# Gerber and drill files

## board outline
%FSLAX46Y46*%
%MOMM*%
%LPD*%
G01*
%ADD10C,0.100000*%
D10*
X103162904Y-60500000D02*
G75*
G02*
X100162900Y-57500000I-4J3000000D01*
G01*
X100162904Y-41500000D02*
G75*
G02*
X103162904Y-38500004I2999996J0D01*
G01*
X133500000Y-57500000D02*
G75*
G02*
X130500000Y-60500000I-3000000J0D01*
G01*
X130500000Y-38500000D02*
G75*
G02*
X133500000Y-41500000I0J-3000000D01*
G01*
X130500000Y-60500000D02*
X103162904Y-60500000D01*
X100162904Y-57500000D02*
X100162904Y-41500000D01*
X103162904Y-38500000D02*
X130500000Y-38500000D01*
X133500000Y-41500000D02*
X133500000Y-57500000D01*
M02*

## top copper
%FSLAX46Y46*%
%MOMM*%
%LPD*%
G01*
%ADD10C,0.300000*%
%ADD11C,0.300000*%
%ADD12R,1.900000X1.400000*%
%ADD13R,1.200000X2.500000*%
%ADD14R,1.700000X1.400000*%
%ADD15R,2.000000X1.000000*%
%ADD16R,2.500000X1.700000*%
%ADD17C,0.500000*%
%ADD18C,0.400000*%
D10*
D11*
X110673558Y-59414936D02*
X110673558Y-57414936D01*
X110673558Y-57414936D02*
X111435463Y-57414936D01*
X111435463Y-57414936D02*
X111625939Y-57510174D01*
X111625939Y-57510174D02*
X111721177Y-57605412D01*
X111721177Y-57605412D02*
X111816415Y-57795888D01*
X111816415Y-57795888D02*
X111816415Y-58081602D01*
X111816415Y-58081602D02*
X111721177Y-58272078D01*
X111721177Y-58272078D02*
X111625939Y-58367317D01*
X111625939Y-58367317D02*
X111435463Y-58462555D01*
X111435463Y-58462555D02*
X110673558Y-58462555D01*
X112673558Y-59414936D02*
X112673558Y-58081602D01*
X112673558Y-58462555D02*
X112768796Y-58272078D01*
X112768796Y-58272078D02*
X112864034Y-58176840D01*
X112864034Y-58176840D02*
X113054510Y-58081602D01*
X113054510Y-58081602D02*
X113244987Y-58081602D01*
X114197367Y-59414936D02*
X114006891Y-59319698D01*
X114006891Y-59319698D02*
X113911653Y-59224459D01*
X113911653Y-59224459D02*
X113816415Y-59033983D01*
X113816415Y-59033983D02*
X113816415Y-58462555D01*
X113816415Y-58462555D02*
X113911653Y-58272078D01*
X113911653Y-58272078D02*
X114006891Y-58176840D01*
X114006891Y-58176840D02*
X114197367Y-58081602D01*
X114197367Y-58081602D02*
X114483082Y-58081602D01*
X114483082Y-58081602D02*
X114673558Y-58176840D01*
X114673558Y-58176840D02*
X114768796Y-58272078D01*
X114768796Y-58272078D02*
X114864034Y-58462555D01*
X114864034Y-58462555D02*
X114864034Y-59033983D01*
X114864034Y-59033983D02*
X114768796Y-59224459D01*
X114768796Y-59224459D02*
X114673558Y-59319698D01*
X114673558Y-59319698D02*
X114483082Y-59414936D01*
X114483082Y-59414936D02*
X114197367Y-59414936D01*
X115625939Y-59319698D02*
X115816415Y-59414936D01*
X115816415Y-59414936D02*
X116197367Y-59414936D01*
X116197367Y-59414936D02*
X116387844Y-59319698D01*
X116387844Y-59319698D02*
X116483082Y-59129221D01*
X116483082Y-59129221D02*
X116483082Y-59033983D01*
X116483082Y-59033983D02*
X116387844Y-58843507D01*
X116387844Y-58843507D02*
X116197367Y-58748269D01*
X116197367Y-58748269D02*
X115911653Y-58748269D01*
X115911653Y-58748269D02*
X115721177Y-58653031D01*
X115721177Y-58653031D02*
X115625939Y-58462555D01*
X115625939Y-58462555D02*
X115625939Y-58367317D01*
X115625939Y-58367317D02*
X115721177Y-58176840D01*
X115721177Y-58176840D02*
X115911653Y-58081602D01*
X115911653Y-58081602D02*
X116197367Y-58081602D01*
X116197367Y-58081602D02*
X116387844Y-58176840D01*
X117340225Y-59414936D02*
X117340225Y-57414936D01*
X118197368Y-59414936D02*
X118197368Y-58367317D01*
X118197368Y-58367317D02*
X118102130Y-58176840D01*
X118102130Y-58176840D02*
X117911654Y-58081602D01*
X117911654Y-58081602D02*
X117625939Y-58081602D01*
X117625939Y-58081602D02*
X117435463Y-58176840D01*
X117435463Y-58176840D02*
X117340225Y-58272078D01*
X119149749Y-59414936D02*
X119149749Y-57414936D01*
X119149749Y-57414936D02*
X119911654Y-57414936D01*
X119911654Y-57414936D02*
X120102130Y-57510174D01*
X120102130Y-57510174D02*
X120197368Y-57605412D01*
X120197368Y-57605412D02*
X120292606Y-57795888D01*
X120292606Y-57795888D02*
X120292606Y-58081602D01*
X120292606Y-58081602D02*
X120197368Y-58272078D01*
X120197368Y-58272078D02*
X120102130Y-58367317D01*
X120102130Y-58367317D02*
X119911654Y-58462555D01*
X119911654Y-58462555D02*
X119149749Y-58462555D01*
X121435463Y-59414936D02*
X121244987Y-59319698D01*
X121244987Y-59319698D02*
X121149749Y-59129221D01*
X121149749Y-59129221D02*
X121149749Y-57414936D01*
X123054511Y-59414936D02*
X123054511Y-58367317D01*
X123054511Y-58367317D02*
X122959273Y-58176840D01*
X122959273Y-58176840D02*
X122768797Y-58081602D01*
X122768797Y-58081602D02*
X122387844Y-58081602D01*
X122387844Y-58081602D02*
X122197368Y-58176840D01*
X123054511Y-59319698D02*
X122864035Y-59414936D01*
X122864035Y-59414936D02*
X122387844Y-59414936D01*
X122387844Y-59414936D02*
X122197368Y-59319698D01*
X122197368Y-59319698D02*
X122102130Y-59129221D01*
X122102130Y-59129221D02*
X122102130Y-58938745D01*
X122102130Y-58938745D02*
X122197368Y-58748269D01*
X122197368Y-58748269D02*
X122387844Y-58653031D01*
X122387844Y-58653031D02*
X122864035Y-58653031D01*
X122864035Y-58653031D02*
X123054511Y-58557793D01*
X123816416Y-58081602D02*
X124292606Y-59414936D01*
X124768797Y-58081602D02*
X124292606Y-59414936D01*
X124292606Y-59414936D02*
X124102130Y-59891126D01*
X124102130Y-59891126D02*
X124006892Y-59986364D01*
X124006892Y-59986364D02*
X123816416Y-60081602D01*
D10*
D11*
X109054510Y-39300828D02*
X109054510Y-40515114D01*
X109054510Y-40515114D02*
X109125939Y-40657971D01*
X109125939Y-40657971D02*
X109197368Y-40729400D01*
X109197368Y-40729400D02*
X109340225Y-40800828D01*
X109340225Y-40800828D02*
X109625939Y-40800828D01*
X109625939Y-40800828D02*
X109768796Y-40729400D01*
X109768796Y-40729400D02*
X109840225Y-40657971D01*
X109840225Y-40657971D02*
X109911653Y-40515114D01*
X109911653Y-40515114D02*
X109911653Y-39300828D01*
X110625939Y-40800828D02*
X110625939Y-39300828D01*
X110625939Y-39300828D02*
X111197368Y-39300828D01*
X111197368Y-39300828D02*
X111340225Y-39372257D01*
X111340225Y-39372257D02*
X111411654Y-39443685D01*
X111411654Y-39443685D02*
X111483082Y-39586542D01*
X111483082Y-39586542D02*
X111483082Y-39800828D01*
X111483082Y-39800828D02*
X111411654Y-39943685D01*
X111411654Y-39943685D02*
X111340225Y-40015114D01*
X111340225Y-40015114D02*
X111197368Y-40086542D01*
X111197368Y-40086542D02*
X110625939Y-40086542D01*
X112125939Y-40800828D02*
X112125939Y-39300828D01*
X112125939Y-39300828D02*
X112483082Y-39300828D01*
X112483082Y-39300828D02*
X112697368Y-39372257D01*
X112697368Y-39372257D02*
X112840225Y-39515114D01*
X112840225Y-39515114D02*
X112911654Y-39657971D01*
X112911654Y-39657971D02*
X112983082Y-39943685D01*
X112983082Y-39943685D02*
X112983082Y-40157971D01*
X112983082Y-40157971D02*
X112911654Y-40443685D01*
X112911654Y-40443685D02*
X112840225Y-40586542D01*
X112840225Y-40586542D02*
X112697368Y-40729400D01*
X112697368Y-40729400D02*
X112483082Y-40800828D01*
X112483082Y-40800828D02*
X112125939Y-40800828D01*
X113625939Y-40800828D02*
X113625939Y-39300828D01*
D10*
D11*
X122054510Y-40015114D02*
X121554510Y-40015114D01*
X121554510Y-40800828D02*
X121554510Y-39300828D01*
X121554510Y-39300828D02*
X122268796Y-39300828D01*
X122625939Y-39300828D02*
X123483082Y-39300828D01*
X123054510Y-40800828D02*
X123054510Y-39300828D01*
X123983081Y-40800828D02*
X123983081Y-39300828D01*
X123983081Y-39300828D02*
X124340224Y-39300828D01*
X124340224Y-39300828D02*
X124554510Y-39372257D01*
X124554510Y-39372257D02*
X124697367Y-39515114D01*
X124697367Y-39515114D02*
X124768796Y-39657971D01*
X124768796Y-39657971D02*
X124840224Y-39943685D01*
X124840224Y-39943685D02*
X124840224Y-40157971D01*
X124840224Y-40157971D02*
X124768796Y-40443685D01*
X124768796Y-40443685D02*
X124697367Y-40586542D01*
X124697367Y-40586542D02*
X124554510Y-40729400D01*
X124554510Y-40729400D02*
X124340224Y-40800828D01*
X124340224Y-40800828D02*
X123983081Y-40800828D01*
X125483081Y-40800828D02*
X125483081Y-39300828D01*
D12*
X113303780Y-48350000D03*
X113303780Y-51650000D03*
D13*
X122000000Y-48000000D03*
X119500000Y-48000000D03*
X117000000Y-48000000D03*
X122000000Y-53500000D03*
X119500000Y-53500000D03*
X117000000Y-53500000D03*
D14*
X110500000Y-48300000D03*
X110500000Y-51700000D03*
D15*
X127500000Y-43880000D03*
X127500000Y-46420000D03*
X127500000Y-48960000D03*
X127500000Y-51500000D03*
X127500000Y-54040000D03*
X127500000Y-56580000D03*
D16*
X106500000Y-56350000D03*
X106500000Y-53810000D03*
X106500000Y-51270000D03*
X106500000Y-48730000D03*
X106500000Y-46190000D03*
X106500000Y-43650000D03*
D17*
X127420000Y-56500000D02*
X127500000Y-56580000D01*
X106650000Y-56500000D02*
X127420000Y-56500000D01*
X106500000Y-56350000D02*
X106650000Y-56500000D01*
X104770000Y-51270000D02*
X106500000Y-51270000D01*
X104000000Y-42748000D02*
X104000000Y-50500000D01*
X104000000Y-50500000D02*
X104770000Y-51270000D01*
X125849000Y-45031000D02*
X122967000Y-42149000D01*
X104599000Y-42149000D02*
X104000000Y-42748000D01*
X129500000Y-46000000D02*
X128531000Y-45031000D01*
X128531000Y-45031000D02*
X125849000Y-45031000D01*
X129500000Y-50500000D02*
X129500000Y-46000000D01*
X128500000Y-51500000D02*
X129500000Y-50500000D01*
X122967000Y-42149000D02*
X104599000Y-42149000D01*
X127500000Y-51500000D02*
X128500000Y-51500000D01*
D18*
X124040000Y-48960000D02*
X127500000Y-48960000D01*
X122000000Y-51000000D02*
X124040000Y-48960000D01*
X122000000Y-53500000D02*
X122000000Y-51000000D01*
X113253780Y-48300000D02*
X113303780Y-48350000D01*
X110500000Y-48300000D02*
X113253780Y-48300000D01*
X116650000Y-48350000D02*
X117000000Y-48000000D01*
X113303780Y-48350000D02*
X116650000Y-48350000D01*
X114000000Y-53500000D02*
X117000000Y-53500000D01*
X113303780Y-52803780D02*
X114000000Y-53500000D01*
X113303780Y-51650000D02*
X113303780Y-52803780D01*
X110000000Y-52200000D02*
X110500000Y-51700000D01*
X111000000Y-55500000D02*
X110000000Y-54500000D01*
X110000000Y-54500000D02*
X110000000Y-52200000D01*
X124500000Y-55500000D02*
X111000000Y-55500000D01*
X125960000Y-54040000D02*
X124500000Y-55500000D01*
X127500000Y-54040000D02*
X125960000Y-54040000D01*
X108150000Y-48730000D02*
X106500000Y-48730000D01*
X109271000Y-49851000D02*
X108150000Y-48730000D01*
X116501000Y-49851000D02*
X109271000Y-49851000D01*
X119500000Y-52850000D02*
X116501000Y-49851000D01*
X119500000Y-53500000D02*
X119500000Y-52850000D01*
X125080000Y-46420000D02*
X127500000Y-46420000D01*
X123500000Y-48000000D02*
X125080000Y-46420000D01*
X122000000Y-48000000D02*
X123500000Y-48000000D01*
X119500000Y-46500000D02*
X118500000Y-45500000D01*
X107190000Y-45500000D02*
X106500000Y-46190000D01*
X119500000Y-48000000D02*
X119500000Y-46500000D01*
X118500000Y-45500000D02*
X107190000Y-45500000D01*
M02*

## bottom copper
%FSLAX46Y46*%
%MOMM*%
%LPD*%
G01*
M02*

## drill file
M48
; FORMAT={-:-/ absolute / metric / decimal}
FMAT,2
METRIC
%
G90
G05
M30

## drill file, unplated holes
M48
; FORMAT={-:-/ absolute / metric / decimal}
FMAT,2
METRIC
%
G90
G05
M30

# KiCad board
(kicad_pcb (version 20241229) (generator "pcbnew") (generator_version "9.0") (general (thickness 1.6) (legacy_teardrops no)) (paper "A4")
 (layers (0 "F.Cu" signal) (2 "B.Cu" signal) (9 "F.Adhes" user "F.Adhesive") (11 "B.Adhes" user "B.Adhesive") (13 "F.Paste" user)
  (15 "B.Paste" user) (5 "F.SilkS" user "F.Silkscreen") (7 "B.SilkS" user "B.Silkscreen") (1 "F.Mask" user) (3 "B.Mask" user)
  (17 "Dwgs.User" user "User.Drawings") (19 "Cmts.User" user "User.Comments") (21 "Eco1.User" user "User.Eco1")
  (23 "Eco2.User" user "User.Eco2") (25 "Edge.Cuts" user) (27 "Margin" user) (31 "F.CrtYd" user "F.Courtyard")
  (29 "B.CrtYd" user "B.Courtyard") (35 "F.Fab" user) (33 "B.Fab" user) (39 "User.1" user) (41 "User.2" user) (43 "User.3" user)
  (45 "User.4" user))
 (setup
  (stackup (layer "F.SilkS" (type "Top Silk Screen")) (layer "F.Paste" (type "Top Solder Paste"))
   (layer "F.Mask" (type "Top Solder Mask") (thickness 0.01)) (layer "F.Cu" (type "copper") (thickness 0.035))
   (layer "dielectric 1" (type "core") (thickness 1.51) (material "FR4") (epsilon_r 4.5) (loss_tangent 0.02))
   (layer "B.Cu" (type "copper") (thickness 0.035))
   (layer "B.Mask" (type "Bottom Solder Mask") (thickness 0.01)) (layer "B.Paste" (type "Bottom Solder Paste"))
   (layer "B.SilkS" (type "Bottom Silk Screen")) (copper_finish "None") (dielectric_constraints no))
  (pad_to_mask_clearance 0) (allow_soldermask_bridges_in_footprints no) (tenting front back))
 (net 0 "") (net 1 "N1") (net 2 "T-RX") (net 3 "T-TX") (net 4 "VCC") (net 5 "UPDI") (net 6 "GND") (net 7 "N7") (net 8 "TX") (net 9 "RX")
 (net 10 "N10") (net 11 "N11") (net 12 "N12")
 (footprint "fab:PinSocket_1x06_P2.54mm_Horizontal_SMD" (layer "F.Cu") (at 127.5 43.88)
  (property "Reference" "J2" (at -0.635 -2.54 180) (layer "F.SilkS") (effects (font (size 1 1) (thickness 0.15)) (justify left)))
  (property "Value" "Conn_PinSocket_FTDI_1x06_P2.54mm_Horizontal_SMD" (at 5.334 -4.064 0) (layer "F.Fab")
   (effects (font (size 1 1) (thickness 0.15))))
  (pad "1" smd rect (at 0 0) (size 2 1) (layers "F.Cu" "F.Mask" "F.Paste") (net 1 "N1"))
  (pad "2" smd rect (at 0 2.54) (size 2 1) (layers "F.Cu" "F.Mask" "F.Paste") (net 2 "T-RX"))
  (pad "3" smd rect (at 0 5.08) (size 2 1) (layers "F.Cu" "F.Mask" "F.Paste") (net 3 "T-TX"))
  (pad "4" smd rect (at 0 7.62) (size 2 1) (layers "F.Cu" "F.Mask" "F.Paste") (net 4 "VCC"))
  (pad "5" smd rect (at 0 10.16) (size 2 1) (layers "F.Cu" "F.Mask" "F.Paste") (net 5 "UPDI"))
  (pad "6" smd rect (at 0 12.7) (size 2 1) (layers "F.Cu" "F.Mask" "F.Paste") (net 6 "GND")))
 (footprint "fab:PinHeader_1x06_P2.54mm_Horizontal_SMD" (layer "F.Cu") (at 106.5 56.35 180)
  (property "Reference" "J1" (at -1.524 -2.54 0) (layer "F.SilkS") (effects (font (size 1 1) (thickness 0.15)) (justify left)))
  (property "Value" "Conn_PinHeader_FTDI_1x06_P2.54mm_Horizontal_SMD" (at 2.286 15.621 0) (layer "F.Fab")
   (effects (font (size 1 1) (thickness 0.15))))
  (pad "1" smd rect (at 0 0 180) (size 2.5 1.7) (layers "F.Cu" "F.Mask" "F.Paste") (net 6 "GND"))
  (pad "2" smd rect (at 0 2.54 180) (size 2.5 1.7) (layers "F.Cu" "F.Mask" "F.Paste") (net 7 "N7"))
  (pad "3" smd rect (at 0 5.08 180) (size 2.5 1.7) (layers "F.Cu" "F.Mask" "F.Paste") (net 4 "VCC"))
  (pad "4" smd rect (at 0 7.62 180) (size 2.5 1.7) (layers "F.Cu" "F.Mask" "F.Paste") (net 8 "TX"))
  (pad "5" smd rect (at 0 10.16 180) (size 2.5 1.7) (layers "F.Cu" "F.Mask" "F.Paste") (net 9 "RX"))
  (pad "6" smd rect (at 0 12.7 180) (size 2.5 1.7) (layers "F.Cu" "F.Mask" "F.Paste") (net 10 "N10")))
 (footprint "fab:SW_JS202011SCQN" (layer "F.Cu") (at 119.5 50.75)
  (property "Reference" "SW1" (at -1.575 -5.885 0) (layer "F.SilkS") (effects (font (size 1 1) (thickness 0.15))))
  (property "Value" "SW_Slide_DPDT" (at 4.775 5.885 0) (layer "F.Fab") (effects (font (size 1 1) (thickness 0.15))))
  (pad "1" smd rect (at -2.5 2.75) (size 1.2 2.5) (layers "F.Cu" "F.Mask" "F.Paste") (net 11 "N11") (solder_mask_margin 0.102))
  (pad "2" smd rect (at 0 2.75) (size 1.2 2.5) (layers "F.Cu" "F.Mask" "F.Paste") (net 8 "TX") (solder_mask_margin 0.102))
  (pad "3" smd rect (at 2.5 2.75) (size 1.2 2.5) (layers "F.Cu" "F.Mask" "F.Paste") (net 3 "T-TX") (solder_mask_margin 0.102))
  (pad "4" smd rect (at 2.5 -2.75) (size 1.2 2.5) (layers "F.Cu" "F.Mask" "F.Paste") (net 2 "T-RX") (solder_mask_margin 0.102))
  (pad "5" smd rect (at 0 -2.75) (size 1.2 2.5) (layers "F.Cu" "F.Mask" "F.Paste") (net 9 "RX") (solder_mask_margin 0.102))
  (pad "6" smd rect (at -2.5 -2.75) (size 1.2 2.5) (layers "F.Cu" "F.Mask" "F.Paste") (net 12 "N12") (solder_mask_margin 0.102)))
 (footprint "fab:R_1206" (layer "F.Cu") (at 110.5 50 -90)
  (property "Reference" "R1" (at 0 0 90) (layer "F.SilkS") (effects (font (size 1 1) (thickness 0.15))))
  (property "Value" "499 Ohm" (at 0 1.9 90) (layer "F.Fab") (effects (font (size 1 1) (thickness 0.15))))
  (pad "1" smd rect (at -1.7 0 270) (size 1.4 1.7) (layers "F.Cu" "F.Mask" "F.Paste") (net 12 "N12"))
  (pad "2" smd rect (at 1.7 0 270) (size 1.4 1.7) (layers "F.Cu" "F.Mask" "F.Paste") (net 5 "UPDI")))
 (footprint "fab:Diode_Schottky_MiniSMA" (layer "F.Cu") (at 113.30378 50 90)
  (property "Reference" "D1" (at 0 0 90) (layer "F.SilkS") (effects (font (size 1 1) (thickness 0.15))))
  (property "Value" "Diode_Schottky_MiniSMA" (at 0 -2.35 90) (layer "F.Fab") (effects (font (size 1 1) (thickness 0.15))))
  (pad "1" smd rect (at -1.65 0 90) (size 1.4 1.9) (layers "F.Cu" "F.Mask" "F.Paste") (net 11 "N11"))
  (pad "2" smd rect (at 1.65 0 90) (size 1.4 1.9) (layers "F.Cu" "F.Mask" "F.Paste") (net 12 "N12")))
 (gr_line (start 103.162904 38.5) (end 130.5 38.5) (stroke (width 0.1) (type default)) (layer "Edge.Cuts"))
 (gr_line (start 130.5 60.5) (end 103.162904 60.5) (stroke (width 0.1) (type default)) (layer "Edge.Cuts"))
 (gr_line (start 100.162904 57.5) (end 100.162904 41.5) (stroke (width 0.1) (type default)) (layer "Edge.Cuts"))
 (gr_arc (start 133.5 57.5) (mid 132.62132 59.62132) (end 130.5 60.5) (stroke (width 0.1) (type default)) (layer "Edge.Cuts"))
 (gr_line (start 133.5 41.5) (end 133.5 57.5) (stroke (width 0.1) (type default)) (layer "Edge.Cuts"))
 (gr_arc (start 100.162904 41.5) (mid 101.041584 39.378681) (end 103.162904 38.5) (stroke (width 0.1) (type default)) (layer "Edge.Cuts"))
 (gr_arc (start 130.5 38.5) (mid 132.62132 39.37868) (end 133.5 41.5) (stroke (width 0.1) (type default)) (layer "Edge.Cuts"))
 (gr_arc (start 103.162904 60.5) (mid 101.041581 59.621322) (end 100.162904 57.5) (stroke (width 0.1) (type default)) (layer "Edge.Cuts"))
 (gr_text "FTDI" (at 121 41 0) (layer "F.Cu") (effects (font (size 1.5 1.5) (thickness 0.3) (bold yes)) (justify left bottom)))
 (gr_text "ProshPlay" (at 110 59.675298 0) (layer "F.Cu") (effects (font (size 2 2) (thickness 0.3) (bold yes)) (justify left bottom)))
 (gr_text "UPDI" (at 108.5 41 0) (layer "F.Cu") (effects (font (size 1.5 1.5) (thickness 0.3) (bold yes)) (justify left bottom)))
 (segment (start 113.30378 48.35) (end 116.65 48.35) (width 0.4) (layer "F.Cu") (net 12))
 (segment (start 113.25378 48.3) (end 113.30378 48.35) (width 0.4) (layer "F.Cu") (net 12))
 (segment (start 116.65 48.35) (end 117 48) (width 0.4) (layer "F.Cu") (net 12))
 (segment (start 110.5 48.3) (end 113.25378 48.3) (width 0.4) (layer "F.Cu") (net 12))
 (segment (start 113.30378 52.80378) (end 114 53.5) (width 0.4) (layer "F.Cu") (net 11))
 (segment (start 113.30378 51.65) (end 113.30378 52.80378) (width 0.4) (layer "F.Cu") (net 11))
 (segment (start 114 53.5) (end 117 53.5) (width 0.4) (layer "F.Cu") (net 11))
 (segment (start 127.42 56.5) (end 127.5 56.58) (width 0.5) (layer "F.Cu") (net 6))
 (segment (start 106.5 56.35) (end 106.65 56.5) (width 0.5) (layer "F.Cu") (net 6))
 (segment (start 106.65 56.5) (end 127.42 56.5) (width 0.5) (layer "F.Cu") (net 6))
 (segment (start 119.5 48) (end 119.5 46.5) (width 0.4) (layer "F.Cu") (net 9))
 (segment (start 107.19 45.5) (end 106.5 46.19) (width 0.4) (layer "F.Cu") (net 9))
 (segment (start 118.5 45.5) (end 107.19 45.5) (width 0.4) (layer "F.Cu") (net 9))
 (segment (start 119.5 46.5) (end 118.5 45.5) (width 0.4) (layer "F.Cu") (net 9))
 (segment (start 104 42.748) (end 104 50.5) (width 0.5) (layer "F.Cu") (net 4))
 (segment (start 129.5 50.5) (end 129.5 46) (width 0.5) (layer "F.Cu") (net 4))
 (segment (start 104 50.5) (end 104.77 51.27) (width 0.5) (layer "F.Cu") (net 4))
 (segment (start 128.5 51.5) (end 129.5 50.5) (width 0.5) (layer "F.Cu") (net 4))
 (segment (start 122.967 42.149) (end 104.599 42.149) (width 0.5) (layer "F.Cu") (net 4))
 (segment (start 104.599 42.149) (end 104 42.748) (width 0.5) (layer "F.Cu") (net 4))
 (segment (start 104.77 51.27) (end 106.5 51.27) (width 0.5) (layer "F.Cu") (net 4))
 (segment (start 125.849 45.031) (end 122.967 42.149) (width 0.5) (layer "F.Cu") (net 4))
 (segment (start 129.5 46) (end 128.531 45.031) (width 0.5) (layer "F.Cu") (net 4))
 (segment (start 128.531 45.031) (end 125.849 45.031) (width 0.5) (layer "F.Cu") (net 4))
 (segment (start 127.5 51.5) (end 128.5 51.5) (width 0.5) (layer "F.Cu") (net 4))
 (segment (start 109.271 49.851) (end 108.15 48.73) (width 0.4) (layer "F.Cu") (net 8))
 (segment (start 119.5 52.85) (end 116.501 49.851) (width 0.4) (layer "F.Cu") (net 8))
 (segment (start 108.15 48.73) (end 106.5 48.73) (width 0.4) (layer "F.Cu") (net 8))
 (segment (start 116.501 49.851) (end 109.271 49.851) (width 0.4) (layer "F.Cu") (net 8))
 (segment (start 119.5 53.5) (end 119.5 52.85) (width 0.4) (layer "F.Cu") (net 8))
 (segment (start 125.96 54.04) (end 124.5 55.5) (width 0.4) (layer "F.Cu") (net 5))
 (segment (start 124.5 55.5) (end 111 55.5) (width 0.4) (layer "F.Cu") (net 5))
 (segment (start 110 54.5) (end 110 52.2) (width 0.4) (layer "F.Cu") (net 5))
 (segment (start 127.5 54.04) (end 125.96 54.04) (width 0.4) (layer "F.Cu") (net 5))
 (segment (start 110 52.2) (end 110.5 51.7) (width 0.4) (layer "F.Cu") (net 5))
 (segment (start 111 55.5) (end 110 54.5) (width 0.4) (layer "F.Cu") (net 5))
 (segment (start 124.04 48.96) (end 127.5 48.96) (width 0.4) (layer "F.Cu") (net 3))
 (segment (start 122 53.5) (end 122 51) (width 0.4) (layer "F.Cu") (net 3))
 (segment (start 122 51) (end 124.04 48.96) (width 0.4) (layer "F.Cu") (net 3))
 (segment (start 125.08 46.42) (end 127.5 46.42) (width 0.4) (layer "F.Cu") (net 2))
 (segment (start 122 48) (end 123.5 48) (width 0.4) (layer "F.Cu") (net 2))
 (segment (start 123.5 48) (end 125.08 46.42) (width 0.4) (layer "F.Cu") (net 2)))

